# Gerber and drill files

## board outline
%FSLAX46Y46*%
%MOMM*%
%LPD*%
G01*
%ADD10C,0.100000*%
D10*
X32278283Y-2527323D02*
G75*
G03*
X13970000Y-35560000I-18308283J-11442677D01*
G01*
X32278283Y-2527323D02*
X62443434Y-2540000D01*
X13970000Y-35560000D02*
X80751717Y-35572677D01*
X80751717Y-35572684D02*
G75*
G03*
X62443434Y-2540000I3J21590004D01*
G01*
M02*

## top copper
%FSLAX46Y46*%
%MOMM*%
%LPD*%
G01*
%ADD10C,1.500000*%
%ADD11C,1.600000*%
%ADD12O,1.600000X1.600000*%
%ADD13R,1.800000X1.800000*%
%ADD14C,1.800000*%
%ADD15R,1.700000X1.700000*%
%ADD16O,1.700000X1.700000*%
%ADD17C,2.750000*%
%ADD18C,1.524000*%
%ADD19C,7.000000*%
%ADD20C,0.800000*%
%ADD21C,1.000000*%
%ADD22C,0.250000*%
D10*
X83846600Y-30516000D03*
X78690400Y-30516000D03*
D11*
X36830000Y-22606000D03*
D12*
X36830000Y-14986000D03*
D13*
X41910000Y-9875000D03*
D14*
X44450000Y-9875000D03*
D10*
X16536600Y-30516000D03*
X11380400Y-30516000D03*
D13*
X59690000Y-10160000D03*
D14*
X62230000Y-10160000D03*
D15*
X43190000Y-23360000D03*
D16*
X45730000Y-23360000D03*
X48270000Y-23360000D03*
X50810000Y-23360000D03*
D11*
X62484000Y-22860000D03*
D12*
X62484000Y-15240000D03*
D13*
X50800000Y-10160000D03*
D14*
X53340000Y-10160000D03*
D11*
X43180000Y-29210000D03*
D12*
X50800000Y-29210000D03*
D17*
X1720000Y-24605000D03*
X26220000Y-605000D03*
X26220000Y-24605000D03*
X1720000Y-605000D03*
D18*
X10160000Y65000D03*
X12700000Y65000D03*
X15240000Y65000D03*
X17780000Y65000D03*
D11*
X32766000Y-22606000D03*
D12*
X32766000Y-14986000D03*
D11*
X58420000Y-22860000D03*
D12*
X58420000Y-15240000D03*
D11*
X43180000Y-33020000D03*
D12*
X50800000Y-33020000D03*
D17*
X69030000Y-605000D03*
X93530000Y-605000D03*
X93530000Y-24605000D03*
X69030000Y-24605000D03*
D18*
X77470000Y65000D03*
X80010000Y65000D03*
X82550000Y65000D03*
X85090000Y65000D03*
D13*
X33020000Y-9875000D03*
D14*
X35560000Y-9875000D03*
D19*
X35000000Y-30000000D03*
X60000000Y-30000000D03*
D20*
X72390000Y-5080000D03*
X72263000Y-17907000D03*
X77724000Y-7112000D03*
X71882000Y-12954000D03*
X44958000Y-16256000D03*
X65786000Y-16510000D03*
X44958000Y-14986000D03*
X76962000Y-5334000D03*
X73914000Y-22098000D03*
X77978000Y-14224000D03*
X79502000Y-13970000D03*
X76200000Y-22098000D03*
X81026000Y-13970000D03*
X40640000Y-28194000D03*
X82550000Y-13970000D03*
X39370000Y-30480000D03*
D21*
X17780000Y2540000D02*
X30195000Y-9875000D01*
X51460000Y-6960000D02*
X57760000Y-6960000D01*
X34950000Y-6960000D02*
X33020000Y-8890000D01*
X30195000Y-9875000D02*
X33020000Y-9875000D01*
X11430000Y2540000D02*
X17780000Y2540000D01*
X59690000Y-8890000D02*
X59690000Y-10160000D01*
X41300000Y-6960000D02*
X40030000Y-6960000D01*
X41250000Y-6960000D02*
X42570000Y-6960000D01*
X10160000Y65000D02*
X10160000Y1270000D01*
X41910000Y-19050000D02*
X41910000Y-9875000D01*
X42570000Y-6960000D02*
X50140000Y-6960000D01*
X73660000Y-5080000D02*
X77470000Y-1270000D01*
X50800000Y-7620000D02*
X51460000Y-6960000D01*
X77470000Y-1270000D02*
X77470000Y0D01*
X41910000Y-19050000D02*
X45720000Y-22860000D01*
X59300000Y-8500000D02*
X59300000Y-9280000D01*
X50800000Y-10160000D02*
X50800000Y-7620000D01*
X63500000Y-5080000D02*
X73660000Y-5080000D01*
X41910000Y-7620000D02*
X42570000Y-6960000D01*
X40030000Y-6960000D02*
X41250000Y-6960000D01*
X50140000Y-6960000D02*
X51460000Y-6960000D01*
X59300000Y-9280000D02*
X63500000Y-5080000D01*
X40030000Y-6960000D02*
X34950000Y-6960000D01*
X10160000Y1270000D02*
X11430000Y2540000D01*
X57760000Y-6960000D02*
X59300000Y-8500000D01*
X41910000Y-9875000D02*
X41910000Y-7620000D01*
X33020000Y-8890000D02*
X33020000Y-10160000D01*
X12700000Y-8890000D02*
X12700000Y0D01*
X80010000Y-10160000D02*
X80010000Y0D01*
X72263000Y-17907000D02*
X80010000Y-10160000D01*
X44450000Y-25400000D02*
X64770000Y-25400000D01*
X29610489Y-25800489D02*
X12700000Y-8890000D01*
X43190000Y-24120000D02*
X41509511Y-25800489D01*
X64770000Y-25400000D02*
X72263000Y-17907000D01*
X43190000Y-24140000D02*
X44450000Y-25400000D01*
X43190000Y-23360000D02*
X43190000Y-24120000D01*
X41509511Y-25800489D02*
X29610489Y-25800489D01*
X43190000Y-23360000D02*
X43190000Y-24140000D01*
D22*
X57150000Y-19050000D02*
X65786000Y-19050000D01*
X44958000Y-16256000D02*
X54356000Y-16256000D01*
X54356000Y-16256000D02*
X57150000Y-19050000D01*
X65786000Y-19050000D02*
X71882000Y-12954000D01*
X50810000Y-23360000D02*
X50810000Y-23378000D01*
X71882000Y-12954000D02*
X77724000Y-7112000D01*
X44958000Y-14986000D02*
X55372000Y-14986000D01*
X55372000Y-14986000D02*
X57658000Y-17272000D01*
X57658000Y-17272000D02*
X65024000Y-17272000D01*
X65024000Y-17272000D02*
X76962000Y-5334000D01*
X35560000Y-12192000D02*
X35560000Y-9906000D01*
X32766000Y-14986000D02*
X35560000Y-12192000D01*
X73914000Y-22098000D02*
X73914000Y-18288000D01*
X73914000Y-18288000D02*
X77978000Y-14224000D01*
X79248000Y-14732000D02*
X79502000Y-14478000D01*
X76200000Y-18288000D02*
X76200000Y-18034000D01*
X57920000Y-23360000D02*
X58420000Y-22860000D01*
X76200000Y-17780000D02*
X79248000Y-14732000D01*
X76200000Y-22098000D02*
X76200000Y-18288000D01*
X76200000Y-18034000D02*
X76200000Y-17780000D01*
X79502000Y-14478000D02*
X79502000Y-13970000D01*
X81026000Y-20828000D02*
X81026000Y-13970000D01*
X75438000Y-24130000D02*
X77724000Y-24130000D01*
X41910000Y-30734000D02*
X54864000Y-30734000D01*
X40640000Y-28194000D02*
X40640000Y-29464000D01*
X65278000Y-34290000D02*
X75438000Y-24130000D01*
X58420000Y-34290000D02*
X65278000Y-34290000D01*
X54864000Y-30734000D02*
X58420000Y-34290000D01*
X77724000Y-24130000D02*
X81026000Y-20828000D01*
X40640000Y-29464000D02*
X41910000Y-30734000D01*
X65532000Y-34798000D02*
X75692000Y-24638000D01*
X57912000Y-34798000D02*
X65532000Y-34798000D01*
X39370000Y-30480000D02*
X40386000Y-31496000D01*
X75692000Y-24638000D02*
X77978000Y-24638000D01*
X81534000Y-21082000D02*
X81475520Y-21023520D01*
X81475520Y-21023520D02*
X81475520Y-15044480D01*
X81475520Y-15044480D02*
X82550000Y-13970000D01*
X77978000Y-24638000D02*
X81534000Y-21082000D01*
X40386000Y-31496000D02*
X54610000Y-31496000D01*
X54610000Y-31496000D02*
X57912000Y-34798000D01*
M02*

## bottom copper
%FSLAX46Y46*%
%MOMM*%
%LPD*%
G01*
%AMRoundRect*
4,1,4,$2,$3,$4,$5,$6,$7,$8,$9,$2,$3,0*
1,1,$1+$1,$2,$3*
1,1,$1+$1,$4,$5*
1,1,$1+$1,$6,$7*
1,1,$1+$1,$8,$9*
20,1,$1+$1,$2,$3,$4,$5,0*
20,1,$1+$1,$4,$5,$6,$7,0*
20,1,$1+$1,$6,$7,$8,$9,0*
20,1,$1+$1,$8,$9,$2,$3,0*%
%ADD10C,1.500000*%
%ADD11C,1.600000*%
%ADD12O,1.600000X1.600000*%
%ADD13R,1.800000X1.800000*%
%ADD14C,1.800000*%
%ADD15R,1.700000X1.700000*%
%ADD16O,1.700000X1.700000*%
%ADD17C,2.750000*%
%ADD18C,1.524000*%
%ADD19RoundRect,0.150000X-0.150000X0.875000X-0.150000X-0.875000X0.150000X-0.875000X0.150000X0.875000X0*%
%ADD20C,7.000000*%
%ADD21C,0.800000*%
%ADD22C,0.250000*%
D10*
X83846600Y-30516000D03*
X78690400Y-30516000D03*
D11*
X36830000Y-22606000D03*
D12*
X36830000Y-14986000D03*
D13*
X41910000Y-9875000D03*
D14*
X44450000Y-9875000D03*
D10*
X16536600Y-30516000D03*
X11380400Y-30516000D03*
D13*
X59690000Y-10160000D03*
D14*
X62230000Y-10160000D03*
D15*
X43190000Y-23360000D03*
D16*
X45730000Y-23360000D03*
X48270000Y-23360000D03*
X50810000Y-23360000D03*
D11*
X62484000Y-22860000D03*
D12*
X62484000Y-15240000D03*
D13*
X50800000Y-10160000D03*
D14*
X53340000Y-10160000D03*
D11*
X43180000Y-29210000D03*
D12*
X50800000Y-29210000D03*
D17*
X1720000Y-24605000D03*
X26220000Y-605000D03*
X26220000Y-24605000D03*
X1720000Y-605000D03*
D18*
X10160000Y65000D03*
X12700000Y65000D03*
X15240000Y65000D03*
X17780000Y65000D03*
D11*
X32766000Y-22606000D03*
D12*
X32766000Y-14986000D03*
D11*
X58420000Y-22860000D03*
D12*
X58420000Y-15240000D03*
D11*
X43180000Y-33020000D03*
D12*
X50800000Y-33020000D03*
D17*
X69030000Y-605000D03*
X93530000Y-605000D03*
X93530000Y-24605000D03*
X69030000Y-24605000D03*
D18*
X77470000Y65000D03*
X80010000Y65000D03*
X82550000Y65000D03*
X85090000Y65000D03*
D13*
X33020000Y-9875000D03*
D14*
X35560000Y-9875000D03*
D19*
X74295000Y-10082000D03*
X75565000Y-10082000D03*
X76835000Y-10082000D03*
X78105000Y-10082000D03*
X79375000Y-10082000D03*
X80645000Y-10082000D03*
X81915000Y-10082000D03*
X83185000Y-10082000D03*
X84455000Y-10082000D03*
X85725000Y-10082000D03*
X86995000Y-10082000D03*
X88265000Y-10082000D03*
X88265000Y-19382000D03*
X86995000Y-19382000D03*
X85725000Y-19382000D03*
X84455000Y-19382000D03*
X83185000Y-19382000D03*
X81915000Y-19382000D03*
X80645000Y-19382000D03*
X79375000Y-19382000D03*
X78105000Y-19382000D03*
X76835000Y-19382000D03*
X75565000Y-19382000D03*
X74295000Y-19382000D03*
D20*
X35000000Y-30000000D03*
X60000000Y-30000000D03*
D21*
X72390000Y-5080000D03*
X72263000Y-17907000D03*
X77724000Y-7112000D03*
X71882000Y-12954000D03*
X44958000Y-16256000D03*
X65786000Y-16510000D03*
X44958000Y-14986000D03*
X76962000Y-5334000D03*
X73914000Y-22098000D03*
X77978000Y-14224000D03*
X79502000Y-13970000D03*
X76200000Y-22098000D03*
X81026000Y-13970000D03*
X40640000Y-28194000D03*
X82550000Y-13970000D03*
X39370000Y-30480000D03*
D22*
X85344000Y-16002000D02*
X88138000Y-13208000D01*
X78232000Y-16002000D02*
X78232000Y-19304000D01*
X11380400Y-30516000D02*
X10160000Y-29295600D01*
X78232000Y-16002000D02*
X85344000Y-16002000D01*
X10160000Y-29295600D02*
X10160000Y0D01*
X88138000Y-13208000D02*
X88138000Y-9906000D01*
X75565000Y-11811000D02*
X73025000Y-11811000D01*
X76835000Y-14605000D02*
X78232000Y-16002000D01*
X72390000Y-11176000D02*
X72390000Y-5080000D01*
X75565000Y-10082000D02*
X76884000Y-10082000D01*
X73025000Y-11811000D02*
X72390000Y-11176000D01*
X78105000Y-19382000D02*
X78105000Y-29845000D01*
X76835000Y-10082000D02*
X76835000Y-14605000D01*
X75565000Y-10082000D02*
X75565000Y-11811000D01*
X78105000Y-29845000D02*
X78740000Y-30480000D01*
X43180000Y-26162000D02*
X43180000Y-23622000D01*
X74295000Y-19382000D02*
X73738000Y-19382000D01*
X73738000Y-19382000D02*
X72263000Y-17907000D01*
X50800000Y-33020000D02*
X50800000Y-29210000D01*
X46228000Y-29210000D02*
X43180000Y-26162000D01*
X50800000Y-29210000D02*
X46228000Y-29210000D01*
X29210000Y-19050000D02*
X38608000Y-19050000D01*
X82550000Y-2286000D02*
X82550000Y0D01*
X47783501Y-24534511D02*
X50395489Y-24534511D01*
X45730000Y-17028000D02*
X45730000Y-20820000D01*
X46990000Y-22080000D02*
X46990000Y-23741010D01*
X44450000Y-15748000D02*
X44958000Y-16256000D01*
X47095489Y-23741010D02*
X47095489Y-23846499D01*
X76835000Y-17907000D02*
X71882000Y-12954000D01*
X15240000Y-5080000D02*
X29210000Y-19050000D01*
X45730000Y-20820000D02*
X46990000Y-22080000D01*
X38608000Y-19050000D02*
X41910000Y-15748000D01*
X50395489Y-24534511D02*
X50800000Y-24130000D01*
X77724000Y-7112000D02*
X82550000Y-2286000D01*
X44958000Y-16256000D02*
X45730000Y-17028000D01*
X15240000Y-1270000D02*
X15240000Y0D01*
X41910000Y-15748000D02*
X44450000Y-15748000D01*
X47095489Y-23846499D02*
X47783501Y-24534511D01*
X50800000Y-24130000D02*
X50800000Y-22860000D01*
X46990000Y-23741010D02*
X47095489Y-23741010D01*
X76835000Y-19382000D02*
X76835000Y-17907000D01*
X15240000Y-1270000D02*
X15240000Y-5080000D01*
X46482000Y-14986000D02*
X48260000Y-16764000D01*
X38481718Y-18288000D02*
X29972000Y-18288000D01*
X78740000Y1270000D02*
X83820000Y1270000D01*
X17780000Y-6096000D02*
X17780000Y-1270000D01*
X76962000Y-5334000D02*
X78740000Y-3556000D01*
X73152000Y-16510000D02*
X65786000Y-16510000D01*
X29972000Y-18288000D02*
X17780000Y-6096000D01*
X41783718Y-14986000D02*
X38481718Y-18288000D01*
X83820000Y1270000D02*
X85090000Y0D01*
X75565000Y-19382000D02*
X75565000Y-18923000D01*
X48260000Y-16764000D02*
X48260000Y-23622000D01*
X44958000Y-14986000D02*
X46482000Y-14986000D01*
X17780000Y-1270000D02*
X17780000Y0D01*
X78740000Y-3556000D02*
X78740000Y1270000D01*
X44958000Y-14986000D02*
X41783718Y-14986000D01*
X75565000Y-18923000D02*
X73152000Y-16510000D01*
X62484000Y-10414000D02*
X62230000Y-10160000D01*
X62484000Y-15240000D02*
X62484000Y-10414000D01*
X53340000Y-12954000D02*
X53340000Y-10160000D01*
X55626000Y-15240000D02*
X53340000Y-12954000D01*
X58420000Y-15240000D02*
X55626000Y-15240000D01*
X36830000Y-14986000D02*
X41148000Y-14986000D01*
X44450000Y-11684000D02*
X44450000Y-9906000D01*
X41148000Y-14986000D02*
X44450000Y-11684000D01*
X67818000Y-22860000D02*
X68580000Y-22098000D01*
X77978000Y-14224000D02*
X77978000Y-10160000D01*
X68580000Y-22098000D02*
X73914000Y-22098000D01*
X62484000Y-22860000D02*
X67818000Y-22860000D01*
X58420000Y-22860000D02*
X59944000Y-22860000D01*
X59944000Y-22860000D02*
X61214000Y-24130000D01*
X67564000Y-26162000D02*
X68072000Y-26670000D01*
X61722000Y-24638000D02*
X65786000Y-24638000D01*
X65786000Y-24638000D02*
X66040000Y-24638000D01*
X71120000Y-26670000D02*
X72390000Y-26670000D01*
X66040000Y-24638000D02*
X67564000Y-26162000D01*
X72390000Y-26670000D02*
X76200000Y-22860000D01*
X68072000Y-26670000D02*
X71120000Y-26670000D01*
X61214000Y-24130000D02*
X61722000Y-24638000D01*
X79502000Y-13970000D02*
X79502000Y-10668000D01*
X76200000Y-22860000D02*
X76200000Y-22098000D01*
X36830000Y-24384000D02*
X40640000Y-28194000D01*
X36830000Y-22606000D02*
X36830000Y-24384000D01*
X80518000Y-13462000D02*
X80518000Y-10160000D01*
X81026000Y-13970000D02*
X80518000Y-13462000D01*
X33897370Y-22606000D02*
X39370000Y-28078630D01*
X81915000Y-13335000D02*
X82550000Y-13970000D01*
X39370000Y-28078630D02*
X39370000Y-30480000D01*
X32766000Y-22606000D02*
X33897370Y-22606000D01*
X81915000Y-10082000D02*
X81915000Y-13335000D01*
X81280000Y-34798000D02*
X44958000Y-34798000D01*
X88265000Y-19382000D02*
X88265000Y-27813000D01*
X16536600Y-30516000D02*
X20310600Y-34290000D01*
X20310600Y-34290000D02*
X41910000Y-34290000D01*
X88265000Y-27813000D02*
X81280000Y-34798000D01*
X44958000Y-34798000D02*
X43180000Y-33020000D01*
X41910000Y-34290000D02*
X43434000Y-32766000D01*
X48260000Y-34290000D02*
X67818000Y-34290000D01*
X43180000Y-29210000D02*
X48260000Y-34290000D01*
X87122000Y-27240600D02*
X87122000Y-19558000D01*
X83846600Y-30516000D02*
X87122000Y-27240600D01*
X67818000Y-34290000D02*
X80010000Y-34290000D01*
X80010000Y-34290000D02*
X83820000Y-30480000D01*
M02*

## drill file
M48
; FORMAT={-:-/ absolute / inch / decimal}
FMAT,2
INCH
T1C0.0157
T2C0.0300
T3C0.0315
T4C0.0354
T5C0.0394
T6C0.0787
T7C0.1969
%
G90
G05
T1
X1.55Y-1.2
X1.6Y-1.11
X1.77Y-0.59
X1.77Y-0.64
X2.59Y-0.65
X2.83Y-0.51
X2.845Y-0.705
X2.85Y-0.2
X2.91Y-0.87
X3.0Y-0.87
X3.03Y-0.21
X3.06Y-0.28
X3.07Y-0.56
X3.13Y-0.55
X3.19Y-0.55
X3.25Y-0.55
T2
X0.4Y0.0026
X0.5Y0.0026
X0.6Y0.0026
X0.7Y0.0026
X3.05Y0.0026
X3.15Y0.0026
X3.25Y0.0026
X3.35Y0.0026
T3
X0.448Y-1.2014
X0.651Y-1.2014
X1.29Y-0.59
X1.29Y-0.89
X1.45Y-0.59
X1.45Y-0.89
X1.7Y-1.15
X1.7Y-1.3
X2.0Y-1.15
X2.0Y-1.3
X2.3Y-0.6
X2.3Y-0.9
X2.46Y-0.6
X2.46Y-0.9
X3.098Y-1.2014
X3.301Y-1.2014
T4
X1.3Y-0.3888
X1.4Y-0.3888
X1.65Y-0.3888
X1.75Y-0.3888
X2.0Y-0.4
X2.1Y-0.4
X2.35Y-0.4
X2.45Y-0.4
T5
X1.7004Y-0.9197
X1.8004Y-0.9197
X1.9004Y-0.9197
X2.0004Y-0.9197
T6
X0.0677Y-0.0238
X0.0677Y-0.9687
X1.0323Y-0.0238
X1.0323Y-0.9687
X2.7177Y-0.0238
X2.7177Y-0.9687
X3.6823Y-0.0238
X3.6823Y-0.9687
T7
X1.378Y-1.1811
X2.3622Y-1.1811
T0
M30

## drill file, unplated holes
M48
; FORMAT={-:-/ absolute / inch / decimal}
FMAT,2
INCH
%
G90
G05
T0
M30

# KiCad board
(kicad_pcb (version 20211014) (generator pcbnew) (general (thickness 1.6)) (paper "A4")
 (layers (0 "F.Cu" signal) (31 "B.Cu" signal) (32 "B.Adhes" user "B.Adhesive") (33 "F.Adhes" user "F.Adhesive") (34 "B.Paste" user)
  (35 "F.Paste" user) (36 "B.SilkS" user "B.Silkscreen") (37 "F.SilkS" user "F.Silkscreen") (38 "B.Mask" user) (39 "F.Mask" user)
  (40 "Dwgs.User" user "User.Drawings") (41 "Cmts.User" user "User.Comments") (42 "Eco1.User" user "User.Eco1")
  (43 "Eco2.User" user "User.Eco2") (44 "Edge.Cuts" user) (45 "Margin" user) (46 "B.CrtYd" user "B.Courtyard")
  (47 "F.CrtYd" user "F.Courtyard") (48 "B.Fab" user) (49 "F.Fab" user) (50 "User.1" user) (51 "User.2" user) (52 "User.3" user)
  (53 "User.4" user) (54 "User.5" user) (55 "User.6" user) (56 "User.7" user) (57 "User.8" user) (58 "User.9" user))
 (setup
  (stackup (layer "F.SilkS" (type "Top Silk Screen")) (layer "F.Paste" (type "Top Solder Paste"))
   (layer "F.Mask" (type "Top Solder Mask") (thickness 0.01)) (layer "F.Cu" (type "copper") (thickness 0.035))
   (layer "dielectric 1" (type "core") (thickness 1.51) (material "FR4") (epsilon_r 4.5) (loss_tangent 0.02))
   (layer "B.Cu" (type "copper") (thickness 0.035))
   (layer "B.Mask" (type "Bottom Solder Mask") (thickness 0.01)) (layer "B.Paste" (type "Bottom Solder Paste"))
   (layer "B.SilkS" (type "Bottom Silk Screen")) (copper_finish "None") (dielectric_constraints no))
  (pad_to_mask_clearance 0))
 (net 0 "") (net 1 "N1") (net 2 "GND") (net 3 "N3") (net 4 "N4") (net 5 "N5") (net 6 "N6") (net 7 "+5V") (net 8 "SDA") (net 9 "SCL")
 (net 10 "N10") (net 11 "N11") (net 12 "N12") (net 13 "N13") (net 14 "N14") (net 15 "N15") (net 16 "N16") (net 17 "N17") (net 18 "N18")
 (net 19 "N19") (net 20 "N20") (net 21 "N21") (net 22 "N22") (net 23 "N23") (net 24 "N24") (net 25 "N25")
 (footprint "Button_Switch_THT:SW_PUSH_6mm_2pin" (layer "F.Cu") (at 57.751717 37.68)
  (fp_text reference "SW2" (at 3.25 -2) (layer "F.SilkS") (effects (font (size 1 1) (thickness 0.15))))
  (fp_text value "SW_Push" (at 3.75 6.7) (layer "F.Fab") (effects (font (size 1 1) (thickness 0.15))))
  (pad "1" thru_hole circle (at 5.8166 2.286 90) (size 1.5 1.5) (drill 0.8) (layers *.Cu *.Mask) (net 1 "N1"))
  (pad "2" thru_hole circle (at 0.6604 2.286 90) (size 1.5 1.5) (drill 0.8) (layers *.Cu *.Mask) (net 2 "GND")))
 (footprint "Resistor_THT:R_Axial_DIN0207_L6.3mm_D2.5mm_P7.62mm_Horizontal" (layer "F.Cu") (at 16.551717 32.056 90)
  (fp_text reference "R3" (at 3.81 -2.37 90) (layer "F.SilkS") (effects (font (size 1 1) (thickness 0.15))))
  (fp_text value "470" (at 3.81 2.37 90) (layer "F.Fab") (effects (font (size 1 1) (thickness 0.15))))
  (pad "1" thru_hole circle (at 0 0 90) (size 1.6 1.6) (drill 0.8) (layers *.Cu *.Mask) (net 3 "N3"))
  (pad "2" thru_hole oval (at 7.62 0 90) (size 1.6 1.6) (drill 0.8) (layers *.Cu *.Mask) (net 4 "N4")))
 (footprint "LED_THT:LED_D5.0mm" (layer "F.Cu") (at 21.631717 19.325)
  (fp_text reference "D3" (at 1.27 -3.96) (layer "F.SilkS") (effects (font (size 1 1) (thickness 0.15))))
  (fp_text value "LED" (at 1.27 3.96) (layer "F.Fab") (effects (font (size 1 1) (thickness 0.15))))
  (pad "1" thru_hole rect (at 0 0) (size 1.8 1.8) (drill 0.9) (layers *.Cu *.Mask) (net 2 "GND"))
  (pad "2" thru_hole circle (at 2.54 0) (size 1.8 1.8) (drill 0.9) (layers *.Cu *.Mask) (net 4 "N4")))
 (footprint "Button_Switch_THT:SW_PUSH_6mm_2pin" (layer "F.Cu") (at -9.558283 37.68)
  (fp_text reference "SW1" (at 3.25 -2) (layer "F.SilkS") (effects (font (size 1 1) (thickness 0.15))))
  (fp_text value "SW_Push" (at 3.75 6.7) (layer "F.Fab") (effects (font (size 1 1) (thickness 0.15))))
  (pad "1" thru_hole circle (at 5.8166 2.286 90) (size 1.5 1.5) (drill 0.8) (layers *.Cu *.Mask) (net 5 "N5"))
  (pad "2" thru_hole circle (at 0.6604 2.286 90) (size 1.5 1.5) (drill 0.8) (layers *.Cu *.Mask) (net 2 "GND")))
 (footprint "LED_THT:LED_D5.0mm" (layer "F.Cu") (at 39.411717 19.61)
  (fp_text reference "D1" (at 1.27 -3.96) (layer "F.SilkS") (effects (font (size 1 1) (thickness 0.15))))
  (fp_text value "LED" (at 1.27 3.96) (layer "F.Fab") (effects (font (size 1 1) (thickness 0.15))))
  (pad "1" thru_hole rect (at 0 0) (size 1.8 1.8) (drill 0.9) (layers *.Cu *.Mask) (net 2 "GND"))
  (pad "2" thru_hole circle (at 2.54 0) (size 1.8 1.8) (drill 0.9) (layers *.Cu *.Mask) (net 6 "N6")))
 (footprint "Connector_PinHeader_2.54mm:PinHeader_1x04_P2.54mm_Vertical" (layer "F.Cu") (at 22.911717 32.81 90)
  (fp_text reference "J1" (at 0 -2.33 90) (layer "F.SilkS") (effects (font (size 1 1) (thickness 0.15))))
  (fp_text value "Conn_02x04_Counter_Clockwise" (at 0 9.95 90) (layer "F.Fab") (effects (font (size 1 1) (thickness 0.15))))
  (pad "1" thru_hole rect (at 0 0 90) (size 1.7 1.7) (drill 1) (layers *.Cu *.Mask) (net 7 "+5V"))
  (pad "2" thru_hole oval (at 0 2.54 90) (size 1.7 1.7) (drill 1) (layers *.Cu *.Mask) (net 2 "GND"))
  (pad "3" thru_hole oval (at 0 5.08 90) (size 1.7 1.7) (drill 1) (layers *.Cu *.Mask) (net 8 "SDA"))
  (pad "4" thru_hole oval (at 0 7.62 90) (size 1.7 1.7) (drill 1) (layers *.Cu *.Mask) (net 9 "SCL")))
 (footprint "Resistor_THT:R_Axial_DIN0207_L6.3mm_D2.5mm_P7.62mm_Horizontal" (layer "F.Cu") (at 42.205717 32.31 90)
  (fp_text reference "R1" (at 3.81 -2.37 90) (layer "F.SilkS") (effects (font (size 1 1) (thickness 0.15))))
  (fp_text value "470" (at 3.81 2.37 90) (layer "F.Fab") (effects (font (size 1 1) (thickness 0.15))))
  (pad "1" thru_hole circle (at 0 0 90) (size 1.6 1.6) (drill 0.8) (layers *.Cu *.Mask) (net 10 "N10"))
  (pad "2" thru_hole oval (at 7.62 0 90) (size 1.6 1.6) (drill 0.8) (layers *.Cu *.Mask) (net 6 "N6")))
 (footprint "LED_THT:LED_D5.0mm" (layer "F.Cu") (at 30.521717 19.61)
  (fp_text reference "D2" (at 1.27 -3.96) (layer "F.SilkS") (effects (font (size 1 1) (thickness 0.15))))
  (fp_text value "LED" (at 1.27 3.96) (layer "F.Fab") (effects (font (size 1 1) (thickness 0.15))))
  (pad "1" thru_hole rect (at 0 0) (size 1.8 1.8) (drill 0.9) (layers *.Cu *.Mask) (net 2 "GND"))
  (pad "2" thru_hole circle (at 2.54 0) (size 1.8 1.8) (drill 0.9) (layers *.Cu *.Mask) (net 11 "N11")))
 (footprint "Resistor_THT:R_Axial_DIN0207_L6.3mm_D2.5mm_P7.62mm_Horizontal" (layer "F.Cu") (at 22.901717 38.66)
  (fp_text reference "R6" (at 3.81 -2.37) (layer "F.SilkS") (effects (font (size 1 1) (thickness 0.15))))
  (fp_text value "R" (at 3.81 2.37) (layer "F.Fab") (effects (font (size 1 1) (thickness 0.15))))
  (pad "1" thru_hole circle (at 0 0) (size 1.6 1.6) (drill 0.8) (layers *.Cu *.Mask) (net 1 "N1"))
  (pad "2" thru_hole oval (at 7.62 0) (size 1.6 1.6) (drill 0.8) (layers *.Cu *.Mask) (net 7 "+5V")))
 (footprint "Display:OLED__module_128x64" (layer "F.Cu") (at -6.308283 36.055)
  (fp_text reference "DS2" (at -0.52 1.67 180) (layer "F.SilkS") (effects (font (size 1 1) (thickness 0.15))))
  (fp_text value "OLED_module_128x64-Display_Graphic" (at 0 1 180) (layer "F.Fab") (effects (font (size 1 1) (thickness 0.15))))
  (pad "" thru_hole circle (at -12.25 -2) (size 2.75 2.75) (drill 2) (layers *.Cu *.Mask))
  (pad "" thru_hole circle (at 12.25 -26) (size 2.75 2.75) (drill 2) (layers *.Cu *.Mask))
  (pad "" thru_hole circle (at 12.25 -2) (size 2.75 2.75) (drill 2) (layers *.Cu *.Mask))
  (pad "" thru_hole circle (at -12.25 -26) (size 2.75 2.75) (drill 2) (layers *.Cu *.Mask))
  (pad "1" thru_hole circle (at -3.81 -26.67) (size 1.524 1.524) (drill 0.762) (layers *.Cu *.Mask) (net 2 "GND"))
  (pad "2" thru_hole circle (at -1.27 -26.67) (size 1.524 1.524) (drill 0.762) (layers *.Cu *.Mask) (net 7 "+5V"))
  (pad "3" thru_hole circle (at 1.27 -26.67) (size 1.524 1.524) (drill 0.762) (layers *.Cu *.Mask) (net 9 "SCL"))
  (pad "4" thru_hole circle (at 3.81 -26.67) (size 1.524 1.524) (drill 0.762) (layers *.Cu *.Mask) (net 8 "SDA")))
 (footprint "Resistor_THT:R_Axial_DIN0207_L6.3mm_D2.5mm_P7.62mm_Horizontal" (layer "F.Cu") (at 12.487717 32.056 90)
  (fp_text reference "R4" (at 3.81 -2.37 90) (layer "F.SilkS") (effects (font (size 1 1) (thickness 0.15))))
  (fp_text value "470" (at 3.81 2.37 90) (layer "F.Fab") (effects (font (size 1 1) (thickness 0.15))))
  (pad "1" thru_hole circle (at 0 0 90) (size 1.6 1.6) (drill 0.8) (layers *.Cu *.Mask) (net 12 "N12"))
  (pad "2" thru_hole oval (at 7.62 0 90) (size 1.6 1.6) (drill 0.8) (layers *.Cu *.Mask) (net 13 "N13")))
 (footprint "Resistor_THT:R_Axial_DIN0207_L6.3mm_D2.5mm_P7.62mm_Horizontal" (layer "F.Cu") (at 38.141717 32.31 90)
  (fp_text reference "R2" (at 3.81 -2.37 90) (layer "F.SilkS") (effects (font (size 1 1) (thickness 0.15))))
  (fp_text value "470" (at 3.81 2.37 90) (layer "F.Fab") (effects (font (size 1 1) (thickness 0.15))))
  (pad "1" thru_hole circle (at 0 0 90) (size 1.6 1.6) (drill 0.8) (layers *.Cu *.Mask) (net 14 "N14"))
  (pad "2" thru_hole oval (at 7.62 0 90) (size 1.6 1.6) (drill 0.8) (layers *.Cu *.Mask) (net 11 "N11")))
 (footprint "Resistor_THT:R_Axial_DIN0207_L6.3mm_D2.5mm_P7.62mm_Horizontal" (layer "F.Cu") (at 22.901717 42.47)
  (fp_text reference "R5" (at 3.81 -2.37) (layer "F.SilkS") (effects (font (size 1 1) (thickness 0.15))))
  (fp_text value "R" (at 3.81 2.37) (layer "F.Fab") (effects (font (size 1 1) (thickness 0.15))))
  (pad "1" thru_hole circle (at 0 0) (size 1.6 1.6) (drill 0.8) (layers *.Cu *.Mask) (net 5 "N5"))
  (pad "2" thru_hole oval (at 7.62 0) (size 1.6 1.6) (drill 0.8) (layers *.Cu *.Mask) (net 7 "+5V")))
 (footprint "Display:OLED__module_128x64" (layer "F.Cu") (at 61.001717 36.055)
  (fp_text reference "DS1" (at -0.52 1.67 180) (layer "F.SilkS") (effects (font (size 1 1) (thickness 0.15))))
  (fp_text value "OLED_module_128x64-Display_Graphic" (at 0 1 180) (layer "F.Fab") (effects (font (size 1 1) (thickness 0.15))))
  (pad "" thru_hole circle (at -12.25 -26) (size 2.75 2.75) (drill 2) (layers *.Cu *.Mask))
  (pad "" thru_hole circle (at 12.25 -26) (size 2.75 2.75) (drill 2) (layers *.Cu *.Mask))
  (pad "" thru_hole circle (at 12.25 -2) (size 2.75 2.75) (drill 2) (layers *.Cu *.Mask))
  (pad "" thru_hole circle (at -12.25 -2) (size 2.75 2.75) (drill 2) (layers *.Cu *.Mask))
  (pad "1" thru_hole circle (at -3.81 -26.67) (size 1.524 1.524) (drill 0.762) (layers *.Cu *.Mask) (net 2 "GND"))
  (pad "2" thru_hole circle (at -1.27 -26.67) (size 1.524 1.524) (drill 0.762) (layers *.Cu *.Mask) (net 7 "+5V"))
  (pad "3" thru_hole circle (at 1.27 -26.67) (size 1.524 1.524) (drill 0.762) (layers *.Cu *.Mask) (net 9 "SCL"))
  (pad "4" thru_hole circle (at 3.81 -26.67) (size 1.524 1.524) (drill 0.762) (layers *.Cu *.Mask) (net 8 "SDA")))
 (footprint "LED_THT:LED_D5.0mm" (layer "F.Cu") (at 12.741717 19.325)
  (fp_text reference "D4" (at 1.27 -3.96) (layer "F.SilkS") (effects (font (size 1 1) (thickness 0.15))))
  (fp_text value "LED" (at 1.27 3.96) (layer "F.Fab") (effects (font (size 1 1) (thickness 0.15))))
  (pad "1" thru_hole rect (at 0 0) (size 1.8 1.8) (drill 0.9) (layers *.Cu *.Mask) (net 2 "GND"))
  (pad "2" thru_hole circle (at 2.54 0) (size 1.8 1.8) (drill 0.9) (layers *.Cu *.Mask) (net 13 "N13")))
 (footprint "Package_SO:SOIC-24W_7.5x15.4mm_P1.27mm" (layer "B.Cu") (at 61.001717 24.182 -90)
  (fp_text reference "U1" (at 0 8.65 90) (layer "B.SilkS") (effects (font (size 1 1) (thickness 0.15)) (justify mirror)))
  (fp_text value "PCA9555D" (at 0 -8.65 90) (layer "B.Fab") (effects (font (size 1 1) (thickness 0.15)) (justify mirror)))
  (pad "1" smd roundrect (at -4.65 6.985 270) (size 2.05 0.6) (layers "B.Cu" "B.Paste" "B.Mask") (roundrect_rratio 0.25) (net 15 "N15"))
  (pad "2" smd roundrect (at -4.65 5.715 270) (size 2.05 0.6) (layers "B.Cu" "B.Paste" "B.Mask") (roundrect_rratio 0.25) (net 2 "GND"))
  (pad "3" smd roundrect (at -4.65 4.445 270) (size 2.05 0.6) (layers "B.Cu" "B.Paste" "B.Mask") (roundrect_rratio 0.25) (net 2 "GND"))
  (pad "4" smd roundrect (at -4.65 3.175 270) (size 2.05 0.6) (layers "B.Cu" "B.Paste" "B.Mask") (roundrect_rratio 0.25) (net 10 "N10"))
  (pad "5" smd roundrect (at -4.65 1.905 270) (size 2.05 0.6) (layers "B.Cu" "B.Paste" "B.Mask") (roundrect_rratio 0.25) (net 14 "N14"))
  (pad "6" smd roundrect (at -4.65 0.635 270) (size 2.05 0.6) (layers "B.Cu" "B.Paste" "B.Mask") (roundrect_rratio 0.25) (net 3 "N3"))
  (pad "7" smd roundrect (at -4.65 -0.635 270) (size 2.05 0.6) (layers "B.Cu" "B.Paste" "B.Mask") (roundrect_rratio 0.25) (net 12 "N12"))
  (pad "8" smd roundrect (at -4.65 -1.905 270) (size 2.05 0.6) (layers "B.Cu" "B.Paste" "B.Mask") (roundrect_rratio 0.25) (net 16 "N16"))
  (pad "9" smd roundrect (at -4.65 -3.175 270) (size 2.05 0.6) (layers "B.Cu" "B.Paste" "B.Mask") (roundrect_rratio 0.25) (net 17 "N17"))
  (pad "10" smd roundrect (at -4.65 -4.445 270) (size 2.05 0.6) (layers "B.Cu" "B.Paste" "B.Mask") (roundrect_rratio 0.25) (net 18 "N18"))
  (pad "11" smd roundrect (at -4.65 -5.715 270) (size 2.05 0.6) (layers "B.Cu" "B.Paste" "B.Mask") (roundrect_rratio 0.25) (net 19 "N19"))
  (pad "12" smd roundrect (at -4.65 -6.985 270) (size 2.05 0.6) (layers "B.Cu" "B.Paste" "B.Mask") (roundrect_rratio 0.25) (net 2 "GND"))
  (pad "13" smd roundrect (at 4.65 -6.985 270) (size 2.05 0.6) (layers "B.Cu" "B.Paste" "B.Mask") (roundrect_rratio 0.25) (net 5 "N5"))
  (pad "14" smd roundrect (at 4.65 -5.715 270) (size 2.05 0.6) (layers "B.Cu" "B.Paste" "B.Mask") (roundrect_rratio 0.25) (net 1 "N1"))
  (pad "15" smd roundrect (at 4.65 -4.445 270) (size 2.05 0.6) (layers "B.Cu" "B.Paste" "B.Mask") (roundrect_rratio 0.25) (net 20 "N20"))
  (pad "16" smd roundrect (at 4.65 -3.175 270) (size 2.05 0.6) (layers "B.Cu" "B.Paste" "B.Mask") (roundrect_rratio 0.25) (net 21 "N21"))
  (pad "17" smd roundrect (at 4.65 -1.905 270) (size 2.05 0.6) (layers "B.Cu" "B.Paste" "B.Mask") (roundrect_rratio 0.25) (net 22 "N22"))
  (pad "18" smd roundrect (at 4.65 -0.635 270) (size 2.05 0.6) (layers "B.Cu" "B.Paste" "B.Mask") (roundrect_rratio 0.25) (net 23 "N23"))
  (pad "19" smd roundrect (at 4.65 0.635 270) (size 2.05 0.6) (layers "B.Cu" "B.Paste" "B.Mask") (roundrect_rratio 0.25) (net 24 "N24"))
  (pad "20" smd roundrect (at 4.65 1.905 270) (size 2.05 0.6) (layers "B.Cu" "B.Paste" "B.Mask") (roundrect_rratio 0.25) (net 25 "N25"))
  (pad "21" smd roundrect (at 4.65 3.175 270) (size 2.05 0.6) (layers "B.Cu" "B.Paste" "B.Mask") (roundrect_rratio 0.25) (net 2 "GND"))
  (pad "22" smd roundrect (at 4.65 4.445 270) (size 2.05 0.6) (layers "B.Cu" "B.Paste" "B.Mask") (roundrect_rratio 0.25) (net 9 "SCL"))
  (pad "23" smd roundrect (at 4.65 5.715 270) (size 2.05 0.6) (layers "B.Cu" "B.Paste" "B.Mask") (roundrect_rratio 0.25) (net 8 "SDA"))
  (pad "24" smd roundrect (at 4.65 6.985 270) (size 2.05 0.6) (layers "B.Cu" "B.Paste" "B.Mask") (roundrect_rratio 0.25) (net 7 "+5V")))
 (gr_arc (start -6.308283 45.01) (mid -25.19332 12.953013) (end 12 11.977323) (layer "Edge.Cuts") (width 0.1))
 (gr_line (start 12 11.977323) (end 42.165151 11.99) (layer "Edge.Cuts") (width 0.1))
 (gr_line (start -6.308283 45.01) (end 60.473434 45.022677) (layer "Edge.Cuts") (width 0.1))
 (gr_arc (start 42.165151 11.99) (mid 79.35847 12.96569) (end 60.473434 45.022677) (layer "Edge.Cuts") (width 0.1))
 (via (at 14.721717 39.45) (size 7) (drill 5) (layers "F.Cu" "B.Cu") (free) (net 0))
 (via (at 39.721717 39.45) (size 7) (drill 5) (layers "F.Cu" "B.Cu") (free) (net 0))
 (segment (start -2.498283 6.91) (end 9.916717 19.325) (width 1) (layer "F.Cu") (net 2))
 (segment (start 31.181717 16.41) (end 37.481717 16.41) (width 1) (layer "F.Cu") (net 2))
 (segment (start 14.671717 16.41) (end 12.741717 18.34) (width 1) (layer "F.Cu") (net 2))
 (segment (start 9.916717 19.325) (end 12.741717 19.325) (width 1) (layer "F.Cu") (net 2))
 (segment (start -8.848283 6.91) (end -2.498283 6.91) (width 1) (layer "F.Cu") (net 2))
 (segment (start 39.411717 18.34) (end 39.411717 19.61) (width 1) (layer "F.Cu") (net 2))
 (segment (start 21.021717 16.41) (end 19.751717 16.41) (width 1) (layer "F.Cu") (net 2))
 (segment (start 20.971717 16.41) (end 22.291717 16.41) (width 1) (layer "F.Cu") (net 2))
 (segment (start -10.118283 9.385) (end -10.118283 8.18) (width 1) (layer "F.Cu") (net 2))
 (segment (start 21.631717 28.5) (end 21.631717 19.325) (width 1) (layer "F.Cu") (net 2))
 (segment (start 22.291717 16.41) (end 29.861717 16.41) (width 1) (layer "F.Cu") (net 2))
 (segment (start 53.381717 14.53) (end 57.191717 10.72) (width 1) (layer "F.Cu") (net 2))
 (segment (start 30.521717 17.07) (end 31.181717 16.41) (width 1) (layer "F.Cu") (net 2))
 (segment (start 57.191717 10.72) (end 57.191717 9.45) (width 1) (layer "F.Cu") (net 2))
 (segment (start 21.631717 28.5) (end 25.441717 32.31) (width 1) (layer "F.Cu") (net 2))
 (segment (start 39.021717 17.95) (end 39.021717 18.73) (width 1) (layer "F.Cu") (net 2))
 (segment (start 30.521717 19.61) (end 30.521717 17.07) (width 1) (layer "F.Cu") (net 2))
 (segment (start 43.221717 14.53) (end 53.381717 14.53) (width 1) (layer "F.Cu") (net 2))
 (segment (start 21.631717 17.07) (end 22.291717 16.41) (width 1) (layer "F.Cu") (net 2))
 (segment (start 19.751717 16.41) (end 20.971717 16.41) (width 1) (layer "F.Cu") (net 2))
 (segment (start 29.861717 16.41) (end 31.181717 16.41) (width 1) (layer "F.Cu") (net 2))
 (segment (start 39.021717 18.73) (end 43.221717 14.53) (width 1) (layer "F.Cu") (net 2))
 (segment (start 19.751717 16.41) (end 14.671717 16.41) (width 1) (layer "F.Cu") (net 2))
 (segment (start -10.118283 8.18) (end -8.848283 6.91) (width 1) (layer "F.Cu") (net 2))
 (segment (start 37.481717 16.41) (end 39.021717 17.95) (width 1) (layer "F.Cu") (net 2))
 (segment (start 21.631717 19.325) (end 21.631717 17.07) (width 1) (layer "F.Cu") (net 2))
 (segment (start 12.741717 18.34) (end 12.741717 19.61) (width 1) (layer "F.Cu") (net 2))
 (via (at 52.111717 14.53) (size 0.8) (drill 0.4) (layers "F.Cu" "B.Cu") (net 2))
 (segment (start 65.065717 25.452) (end 67.859717 22.658) (width 0.25) (layer "B.Cu") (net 2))
 (segment (start 57.953717 25.452) (end 57.953717 28.754) (width 0.25) (layer "B.Cu") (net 2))
 (segment (start -8.897883 39.966) (end -10.118283 38.7456) (width 0.25) (layer "B.Cu") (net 2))
 (segment (start 57.953717 25.452) (end 65.065717 25.452) (width 0.25) (layer "B.Cu") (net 2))
 (segment (start -10.118283 38.7456) (end -10.118283 9.45) (width 0.25) (layer "B.Cu") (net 2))
 (segment (start 67.859717 22.658) (end 67.859717 19.356) (width 0.25) (layer "B.Cu") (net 2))
 (segment (start 55.286717 21.261) (end 52.746717 21.261) (width 0.25) (layer "B.Cu") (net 2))
 (segment (start 56.556717 24.055) (end 57.953717 25.452) (width 0.25) (layer "B.Cu") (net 2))
 (segment (start 52.111717 20.626) (end 52.111717 14.53) (width 0.25) (layer "B.Cu") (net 2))
 (segment (start 55.286717 19.532) (end 56.605717 19.532) (width 0.25) (layer "B.Cu") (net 2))
 (segment (start 52.746717 21.261) (end 52.111717 20.626) (width 0.25) (layer "B.Cu") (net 2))
 (segment (start 57.826717 28.832) (end 57.826717 39.295) (width 0.25) (layer "B.Cu") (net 2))
 (segment (start 56.556717 19.532) (end 56.556717 24.055) (width 0.25) (layer "B.Cu") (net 2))
 (segment (start 55.286717 19.532) (end 55.286717 21.261) (width 0.25) (layer "B.Cu") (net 2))
 (segment (start 57.826717 39.295) (end 58.461717 39.93) (width 0.25) (layer "B.Cu") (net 2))
 (segment (start -7.578283 18.34) (end -7.578283 9.45) (width 1) (layer "F.Cu") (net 7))
 (segment (start 59.731717 19.61) (end 59.731717 9.45) (width 1) (layer "F.Cu") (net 7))
 (segment (start 51.984717 27.357) (end 59.731717 19.61) (width 1) (layer "F.Cu") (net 7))
 (segment (start 24.171717 34.85) (end 44.491717 34.85) (width 1) (layer "F.Cu") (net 7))
 (segment (start 9.332206 35.250489) (end -7.578283 18.34) (width 1) (layer "F.Cu") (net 7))
 (segment (start 22.911717 33.57) (end 21.231228 35.250489) (width 1) (layer "F.Cu") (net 7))
 (segment (start 44.491717 34.85) (end 51.984717 27.357) (width 1) (layer "F.Cu") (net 7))
 (segment (start 22.911717 33.59) (end 24.171717 34.85) (width 1) (layer "F.Cu") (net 7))
 (segment (start 22.911717 32.81) (end 22.911717 33.57) (width 1) (layer "F.Cu") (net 7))
 (segment (start 21.231228 35.250489) (end 9.332206 35.250489) (width 1) (layer "F.Cu") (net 7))
 (segment (start 22.911717 32.81) (end 22.911717 33.59) (width 1) (layer "F.Cu") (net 7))
 (via (at 51.984717 27.357) (size 0.8) (drill 0.4) (layers "F.Cu" "B.Cu") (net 7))
 (segment (start 22.901717 35.612) (end 22.901717 33.072) (width 0.25) (layer "B.Cu") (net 7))
 (segment (start 54.016717 28.832) (end 53.459717 28.832) (width 0.25) (layer "B.Cu") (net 7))
 (segment (start 53.459717 28.832) (end 51.984717 27.357) (width 0.25) (layer "B.Cu") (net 7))
 (segment (start 30.521717 42.47) (end 30.521717 38.66) (width 0.25) (layer "B.Cu") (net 7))
 (segment (start 25.949717 38.66) (end 22.901717 35.612) (width 0.25) (layer "B.Cu") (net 7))
 (segment (start 30.521717 38.66) (end 25.949717 38.66) (width 0.25) (layer "B.Cu") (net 7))
 (segment (start 36.871717 28.5) (end 45.507717 28.5) (width 0.25) (layer "F.Cu") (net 9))
 (segment (start 24.679717 25.706) (end 34.077717 25.706) (width 0.25) (layer "F.Cu") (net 9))
 (segment (start 34.077717 25.706) (end 36.871717 28.5) (width 0.25) (layer "F.Cu") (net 9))
 (segment (start 45.507717 28.5) (end 51.603717 22.404) (width 0.25) (layer "F.Cu") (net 9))
 (segment (start 30.531717 32.81) (end 30.531717 32.828) (width 0.25) (layer "F.Cu") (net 9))
 (segment (start 51.603717 22.404) (end 57.445717 16.562) (width 0.25) (layer "F.Cu") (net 9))
 (via (at 57.445717 16.562) (size 0.8) (drill 0.4) (layers "F.Cu" "B.Cu") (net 9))
 (via (at 51.603717 22.404) (size 0.8) (drill 0.4) (layers "F.Cu" "B.Cu") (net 9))
 (via (at 24.679717 25.706) (size 0.8) (drill 0.4) (layers "F.Cu" "B.Cu") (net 9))
 (segment (start 8.931717 28.5) (end 18.329717 28.5) (width 0.25) (layer "B.Cu") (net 9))
 (segment (start 62.271717 11.736) (end 62.271717 9.45) (width 0.25) (layer "B.Cu") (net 9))
 (segment (start 27.505218 33.984511) (end 30.117206 33.984511) (width 0.25) (layer "B.Cu") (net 9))
 (segment (start 25.451717 26.478) (end 25.451717 30.27) (width 0.25) (layer "B.Cu") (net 9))
 (segment (start 26.711717 31.53) (end 26.711717 33.19101) (width 0.25) (layer "B.Cu") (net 9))
 (segment (start 24.171717 25.198) (end 24.679717 25.706) (width 0.25) (layer "B.Cu") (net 9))
 (segment (start 26.817206 33.19101) (end 26.817206 33.296499) (width 0.25) (layer "B.Cu") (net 9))
 (segment (start 56.556717 27.357) (end 51.603717 22.404) (width 0.25) (layer "B.Cu") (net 9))
 (segment (start -5.038283 14.53) (end 8.931717 28.5) (width 0.25) (layer "B.Cu") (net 9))
 (segment (start 25.451717 30.27) (end 26.711717 31.53) (width 0.25) (layer "B.Cu") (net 9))
 (segment (start 18.329717 28.5) (end 21.631717 25.198) (width 0.25) (layer "B.Cu") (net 9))
 (segment (start 30.117206 33.984511) (end 30.521717 33.58) (width 0.25) (layer "B.Cu") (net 9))
 (segment (start 57.445717 16.562) (end 62.271717 11.736) (width 0.25) (layer "B.Cu") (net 9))
 (segment (start 24.679717 25.706) (end 25.451717 26.478) (width 0.25) (layer "B.Cu") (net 9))
 (segment (start -5.038283 10.72) (end -5.038283 9.45) (width 0.25) (layer "B.Cu") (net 9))
 (segment (start 21.631717 25.198) (end 24.171717 25.198) (width 0.25) (layer "B.Cu") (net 9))
 (segment (start 26.817206 33.296499) (end 27.505218 33.984511) (width 0.25) (layer "B.Cu") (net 9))
 (segment (start 30.521717 33.58) (end 30.521717 32.31) (width 0.25) (layer "B.Cu") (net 9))
 (segment (start 26.711717 33.19101) (end 26.817206 33.19101) (width 0.25) (layer "B.Cu") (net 9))
 (segment (start 56.556717 28.832) (end 56.556717 27.357) (width 0.25) (layer "B.Cu") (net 9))
 (segment (start -5.038283 10.72) (end -5.038283 14.53) (width 0.25) (layer "B.Cu") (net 9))
 (segment (start 24.679717 24.436) (end 35.093717 24.436) (width 0.25) (layer "F.Cu") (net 8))
 (segment (start 35.093717 24.436) (end 37.379717 26.722) (width 0.25) (layer "F.Cu") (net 8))
 (segment (start 37.379717 26.722) (end 44.745717 26.722) (width 0.25) (layer "F.Cu") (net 8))
 (segment (start 44.745717 26.722) (end 56.683717 14.784) (width 0.25) (layer "F.Cu") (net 8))
 (via (at 45.507717 25.96) (size 0.8) (drill 0.4) (layers "F.Cu" "B.Cu") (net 8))
 (via (at 24.679717 24.436) (size 0.8) (drill 0.4) (layers "F.Cu" "B.Cu") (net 8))
 (via (at 56.683717 14.784) (size 0.8) (drill 0.4) (layers "F.Cu" "B.Cu") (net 8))
 (segment (start 26.203717 24.436) (end 27.981717 26.214) (width 0.25) (layer "B.Cu") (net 8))
 (segment (start 18.203435 27.738) (end 9.693717 27.738) (width 0.25) (layer "B.Cu") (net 8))
 (segment (start 58.461717 8.18) (end 63.541717 8.18) (width 0.25) (layer "B.Cu") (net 8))
 (segment (start -2.498283 15.546) (end -2.498283 10.72) (width 0.25) (layer "B.Cu") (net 8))
 (segment (start 56.683717 14.784) (end 58.461717 13.006) (width 0.25) (layer "B.Cu") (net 8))
 (segment (start 52.873717 25.96) (end 45.507717 25.96) (width 0.25) (layer "B.Cu") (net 8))
 (segment (start 9.693717 27.738) (end -2.498283 15.546) (width 0.25) (layer "B.Cu") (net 8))
 (segment (start 21.505435 24.436) (end 18.203435 27.738) (width 0.25) (layer "B.Cu") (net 8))
 (segment (start 63.541717 8.18) (end 64.811717 9.45) (width 0.25) (layer "B.Cu") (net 8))
 (segment (start 55.286717 28.832) (end 55.286717 28.373) (width 0.25) (layer "B.Cu") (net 8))
 (segment (start 27.981717 26.214) (end 27.981717 33.072) (width 0.25) (layer "B.Cu") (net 8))
 (segment (start 24.679717 24.436) (end 26.203717 24.436) (width 0.25) (layer "B.Cu") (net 8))
 (segment (start -2.498283 10.72) (end -2.498283 9.45) (width 0.25) (layer "B.Cu") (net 8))
 (segment (start 58.461717 13.006) (end 58.461717 8.18) (width 0.25) (layer "B.Cu") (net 8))
 (segment (start 24.679717 24.436) (end 21.505435 24.436) (width 0.25) (layer "B.Cu") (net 8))
 (segment (start 55.286717 28.373) (end 52.873717 25.96) (width 0.25) (layer "B.Cu") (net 8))
 (segment (start 42.205717 19.864) (end 41.951717 19.61) (width 0.25) (layer "B.Cu") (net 6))
 (segment (start 42.205717 24.69) (end 42.205717 19.864) (width 0.25) (layer "B.Cu") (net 6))
 (segment (start 33.061717 22.404) (end 33.061717 19.61) (width 0.25) (layer "B.Cu") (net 11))
 (segment (start 35.347717 24.69) (end 33.061717 22.404) (width 0.25) (layer "B.Cu") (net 11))
 (segment (start 38.141717 24.69) (end 35.347717 24.69) (width 0.25) (layer "B.Cu") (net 11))
 (segment (start 16.551717 24.436) (end 20.869717 24.436) (width 0.25) (layer "B.Cu") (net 4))
 (segment (start 24.171717 21.134) (end 24.171717 19.356) (width 0.25) (layer "B.Cu") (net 4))
 (segment (start 20.869717 24.436) (end 24.171717 21.134) (width 0.25) (layer "B.Cu") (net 4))
 (segment (start 15.281717 21.642) (end 15.281717 19.356) (width 0.25) (layer "F.Cu") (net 13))
 (segment (start 12.487717 24.436) (end 15.281717 21.642) (width 0.25) (layer "F.Cu") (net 13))
 (segment (start 53.635717 31.548) (end 53.635717 27.738) (width 0.25) (layer "F.Cu") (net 10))
 (segment (start 53.635717 27.738) (end 57.699717 23.674) (width 0.25) (layer "F.Cu") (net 10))
 (via (at 53.635717 31.548) (size 0.8) (drill 0.4) (layers "F.Cu" "B.Cu") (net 10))
 (via (at 57.699717 23.674) (size 0.8) (drill 0.4) (layers "F.Cu" "B.Cu") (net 10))
 (segment (start 47.539717 32.31) (end 48.301717 31.548) (width 0.25) (layer "B.Cu") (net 10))
 (segment (start 57.699717 23.674) (end 57.699717 19.61) (width 0.25) (layer "B.Cu") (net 10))
 (segment (start 48.301717 31.548) (end 53.635717 31.548) (width 0.25) (layer "B.Cu") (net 10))
 (segment (start 42.205717 32.31) (end 47.539717 32.31) (width 0.25) (layer "B.Cu") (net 10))
 (segment (start 58.969717 24.182) (end 59.223717 23.928) (width 0.25) (layer "F.Cu") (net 14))
 (segment (start 55.921717 27.738) (end 55.921717 27.484) (width 0.25) (layer "F.Cu") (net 14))
 (segment (start 37.641717 32.81) (end 38.141717 32.31) (width 0.25) (layer "F.Cu") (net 14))
 (segment (start 55.921717 27.23) (end 58.969717 24.182) (width 0.25) (layer "F.Cu") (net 14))
 (segment (start 55.921717 31.548) (end 55.921717 27.738) (width 0.25) (layer "F.Cu") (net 14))
 (segment (start 55.921717 27.484) (end 55.921717 27.23) (width 0.25) (layer "F.Cu") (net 14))
 (segment (start 59.223717 23.928) (end 59.223717 23.42) (width 0.25) (layer "F.Cu") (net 14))
 (via (at 59.223717 23.42) (size 0.8) (drill 0.4) (layers "F.Cu" "B.Cu") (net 14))
 (via (at 55.921717 31.548) (size 0.8) (drill 0.4) (layers "F.Cu" "B.Cu") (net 14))
 (segment (start 38.141717 32.31) (end 39.665717 32.31) (width 0.25) (layer "B.Cu") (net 14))
 (segment (start 39.665717 32.31) (end 40.935717 33.58) (width 0.25) (layer "B.Cu") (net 14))
 (segment (start 47.285717 35.612) (end 47.793717 36.12) (width 0.25) (layer "B.Cu") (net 14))
 (segment (start 41.443717 34.088) (end 45.507717 34.088) (width 0.25) (layer "B.Cu") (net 14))
 (segment (start 45.507717 34.088) (end 45.761717 34.088) (width 0.25) (layer "B.Cu") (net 14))
 (segment (start 50.841717 36.12) (end 52.111717 36.12) (width 0.25) (layer "B.Cu") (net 14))
 (segment (start 45.761717 34.088) (end 47.285717 35.612) (width 0.25) (layer "B.Cu") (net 14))
 (segment (start 52.111717 36.12) (end 55.921717 32.31) (width 0.25) (layer "B.Cu") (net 14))
 (segment (start 47.793717 36.12) (end 50.841717 36.12) (width 0.25) (layer "B.Cu") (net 14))
 (segment (start 40.935717 33.58) (end 41.443717 34.088) (width 0.25) (layer "B.Cu") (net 14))
 (segment (start 59.223717 23.42) (end 59.223717 20.118) (width 0.25) (layer "B.Cu") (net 14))
 (segment (start 55.921717 32.31) (end 55.921717 31.548) (width 0.25) (layer "B.Cu") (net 14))
 (segment (start 60.747717 30.278) (end 60.747717 23.42) (width 0.25) (layer "F.Cu") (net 3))
 (segment (start 55.159717 33.58) (end 57.445717 33.58) (width 0.25) (layer "F.Cu") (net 3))
 (segment (start 21.631717 40.184) (end 34.585717 40.184) (width 0.25) (layer "F.Cu") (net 3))
 (segment (start 20.361717 37.644) (end 20.361717 38.914) (width 0.25) (layer "F.Cu") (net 3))
 (segment (start 44.999717 43.74) (end 55.159717 33.58) (width 0.25) (layer "F.Cu") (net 3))
 (segment (start 38.141717 43.74) (end 44.999717 43.74) (width 0.25) (layer "F.Cu") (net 3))
 (segment (start 34.585717 40.184) (end 38.141717 43.74) (width 0.25) (layer "F.Cu") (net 3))
 (segment (start 57.445717 33.58) (end 60.747717 30.278) (width 0.25) (layer "F.Cu") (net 3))
 (segment (start 20.361717 38.914) (end 21.631717 40.184) (width 0.25) (layer "F.Cu") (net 3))
 (via (at 60.747717 23.42) (size 0.8) (drill 0.4) (layers "F.Cu" "B.Cu") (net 3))
 (via (at 20.361717 37.644) (size 0.8) (drill 0.4) (layers "F.Cu" "B.Cu") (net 3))
 (segment (start 16.551717 33.834) (end 20.361717 37.644) (width 0.25) (layer "B.Cu") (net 3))
 (segment (start 16.551717 32.056) (end 16.551717 33.834) (width 0.25) (layer "B.Cu") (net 3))
 (segment (start 60.239717 22.912) (end 60.239717 19.61) (width 0.25) (layer "B.Cu") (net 3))
 (segment (start 60.747717 23.42) (end 60.239717 22.912) (width 0.25) (layer "B.Cu") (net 3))
 (segment (start 45.253717 44.248) (end 55.413717 34.088) (width 0.25) (layer "F.Cu") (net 12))
 (segment (start 37.633717 44.248) (end 45.253717 44.248) (width 0.25) (layer "F.Cu") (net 12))
 (segment (start 19.091717 39.93) (end 20.107717 40.946) (width 0.25) (layer "F.Cu") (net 12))
 (segment (start 55.413717 34.088) (end 57.699717 34.088) (width 0.25) (layer "F.Cu") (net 12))
 (segment (start 61.255717 30.532) (end 61.197237 30.47352) (width 0.25) (layer "F.Cu") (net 12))
 (segment (start 61.197237 30.47352) (end 61.197237 24.49448) (width 0.25) (layer "F.Cu") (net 12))
 (segment (start 61.197237 24.49448) (end 62.271717 23.42) (width 0.25) (layer "F.Cu") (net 12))
 (segment (start 57.699717 34.088) (end 61.255717 30.532) (width 0.25) (layer "F.Cu") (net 12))
 (segment (start 20.107717 40.946) (end 34.331717 40.946) (width 0.25) (layer "F.Cu") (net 12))
 (segment (start 34.331717 40.946) (end 37.633717 44.248) (width 0.25) (layer "F.Cu") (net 12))
 (via (at 62.271717 23.42) (size 0.8) (drill 0.4) (layers "F.Cu" "B.Cu") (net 12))
 (via (at 19.091717 39.93) (size 0.8) (drill 0.4) (layers "F.Cu" "B.Cu") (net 12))
 (segment (start 13.619087 32.056) (end 19.091717 37.52863) (width 0.25) (layer "B.Cu") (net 12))
 (segment (start 61.636717 22.785) (end 62.271717 23.42) (width 0.25) (layer "B.Cu") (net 12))
 (segment (start 19.091717 37.52863) (end 19.091717 39.93) (width 0.25) (layer "B.Cu") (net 12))
 (segment (start 12.487717 32.056) (end 13.619087 32.056) (width 0.25) (layer "B.Cu") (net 12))
 (segment (start 61.636717 19.532) (end 61.636717 22.785) (width 0.25) (layer "B.Cu") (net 12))
 (segment (start 61.001717 44.248) (end 24.679717 44.248) (width 0.25) (layer "B.Cu") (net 5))
 (segment (start 67.986717 28.832) (end 67.986717 37.263) (width 0.25) (layer "B.Cu") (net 5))
 (segment (start -3.741683 39.966) (end 0.032317 43.74) (width 0.25) (layer "B.Cu") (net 5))
 (segment (start 0.032317 43.74) (end 21.631717 43.74) (width 0.25) (layer "B.Cu") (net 5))
 (segment (start 67.986717 37.263) (end 61.001717 44.248) (width 0.25) (layer "B.Cu") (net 5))
 (segment (start 24.679717 44.248) (end 22.901717 42.47) (width 0.25) (layer "B.Cu") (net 5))
 (segment (start 21.631717 43.74) (end 23.155717 42.216) (width 0.25) (layer "B.Cu") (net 5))
 (segment (start 27.981717 43.74) (end 47.539717 43.74) (width 0.25) (layer "B.Cu") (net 1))
 (segment (start 22.901717 38.66) (end 27.981717 43.74) (width 0.25) (layer "B.Cu") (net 1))
 (segment (start 66.843717 36.6906) (end 66.843717 29.008) (width 0.25) (layer "B.Cu") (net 1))
 (segment (start 63.568317 39.966) (end 66.843717 36.6906) (width 0.25) (layer "B.Cu") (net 1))
 (segment (start 47.539717 43.74) (end 59.731717 43.74) (width 0.25) (layer "B.Cu") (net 1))
 (segment (start 59.731717 43.74) (end 63.541717 39.93) (width 0.25) (layer "B.Cu") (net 1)))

